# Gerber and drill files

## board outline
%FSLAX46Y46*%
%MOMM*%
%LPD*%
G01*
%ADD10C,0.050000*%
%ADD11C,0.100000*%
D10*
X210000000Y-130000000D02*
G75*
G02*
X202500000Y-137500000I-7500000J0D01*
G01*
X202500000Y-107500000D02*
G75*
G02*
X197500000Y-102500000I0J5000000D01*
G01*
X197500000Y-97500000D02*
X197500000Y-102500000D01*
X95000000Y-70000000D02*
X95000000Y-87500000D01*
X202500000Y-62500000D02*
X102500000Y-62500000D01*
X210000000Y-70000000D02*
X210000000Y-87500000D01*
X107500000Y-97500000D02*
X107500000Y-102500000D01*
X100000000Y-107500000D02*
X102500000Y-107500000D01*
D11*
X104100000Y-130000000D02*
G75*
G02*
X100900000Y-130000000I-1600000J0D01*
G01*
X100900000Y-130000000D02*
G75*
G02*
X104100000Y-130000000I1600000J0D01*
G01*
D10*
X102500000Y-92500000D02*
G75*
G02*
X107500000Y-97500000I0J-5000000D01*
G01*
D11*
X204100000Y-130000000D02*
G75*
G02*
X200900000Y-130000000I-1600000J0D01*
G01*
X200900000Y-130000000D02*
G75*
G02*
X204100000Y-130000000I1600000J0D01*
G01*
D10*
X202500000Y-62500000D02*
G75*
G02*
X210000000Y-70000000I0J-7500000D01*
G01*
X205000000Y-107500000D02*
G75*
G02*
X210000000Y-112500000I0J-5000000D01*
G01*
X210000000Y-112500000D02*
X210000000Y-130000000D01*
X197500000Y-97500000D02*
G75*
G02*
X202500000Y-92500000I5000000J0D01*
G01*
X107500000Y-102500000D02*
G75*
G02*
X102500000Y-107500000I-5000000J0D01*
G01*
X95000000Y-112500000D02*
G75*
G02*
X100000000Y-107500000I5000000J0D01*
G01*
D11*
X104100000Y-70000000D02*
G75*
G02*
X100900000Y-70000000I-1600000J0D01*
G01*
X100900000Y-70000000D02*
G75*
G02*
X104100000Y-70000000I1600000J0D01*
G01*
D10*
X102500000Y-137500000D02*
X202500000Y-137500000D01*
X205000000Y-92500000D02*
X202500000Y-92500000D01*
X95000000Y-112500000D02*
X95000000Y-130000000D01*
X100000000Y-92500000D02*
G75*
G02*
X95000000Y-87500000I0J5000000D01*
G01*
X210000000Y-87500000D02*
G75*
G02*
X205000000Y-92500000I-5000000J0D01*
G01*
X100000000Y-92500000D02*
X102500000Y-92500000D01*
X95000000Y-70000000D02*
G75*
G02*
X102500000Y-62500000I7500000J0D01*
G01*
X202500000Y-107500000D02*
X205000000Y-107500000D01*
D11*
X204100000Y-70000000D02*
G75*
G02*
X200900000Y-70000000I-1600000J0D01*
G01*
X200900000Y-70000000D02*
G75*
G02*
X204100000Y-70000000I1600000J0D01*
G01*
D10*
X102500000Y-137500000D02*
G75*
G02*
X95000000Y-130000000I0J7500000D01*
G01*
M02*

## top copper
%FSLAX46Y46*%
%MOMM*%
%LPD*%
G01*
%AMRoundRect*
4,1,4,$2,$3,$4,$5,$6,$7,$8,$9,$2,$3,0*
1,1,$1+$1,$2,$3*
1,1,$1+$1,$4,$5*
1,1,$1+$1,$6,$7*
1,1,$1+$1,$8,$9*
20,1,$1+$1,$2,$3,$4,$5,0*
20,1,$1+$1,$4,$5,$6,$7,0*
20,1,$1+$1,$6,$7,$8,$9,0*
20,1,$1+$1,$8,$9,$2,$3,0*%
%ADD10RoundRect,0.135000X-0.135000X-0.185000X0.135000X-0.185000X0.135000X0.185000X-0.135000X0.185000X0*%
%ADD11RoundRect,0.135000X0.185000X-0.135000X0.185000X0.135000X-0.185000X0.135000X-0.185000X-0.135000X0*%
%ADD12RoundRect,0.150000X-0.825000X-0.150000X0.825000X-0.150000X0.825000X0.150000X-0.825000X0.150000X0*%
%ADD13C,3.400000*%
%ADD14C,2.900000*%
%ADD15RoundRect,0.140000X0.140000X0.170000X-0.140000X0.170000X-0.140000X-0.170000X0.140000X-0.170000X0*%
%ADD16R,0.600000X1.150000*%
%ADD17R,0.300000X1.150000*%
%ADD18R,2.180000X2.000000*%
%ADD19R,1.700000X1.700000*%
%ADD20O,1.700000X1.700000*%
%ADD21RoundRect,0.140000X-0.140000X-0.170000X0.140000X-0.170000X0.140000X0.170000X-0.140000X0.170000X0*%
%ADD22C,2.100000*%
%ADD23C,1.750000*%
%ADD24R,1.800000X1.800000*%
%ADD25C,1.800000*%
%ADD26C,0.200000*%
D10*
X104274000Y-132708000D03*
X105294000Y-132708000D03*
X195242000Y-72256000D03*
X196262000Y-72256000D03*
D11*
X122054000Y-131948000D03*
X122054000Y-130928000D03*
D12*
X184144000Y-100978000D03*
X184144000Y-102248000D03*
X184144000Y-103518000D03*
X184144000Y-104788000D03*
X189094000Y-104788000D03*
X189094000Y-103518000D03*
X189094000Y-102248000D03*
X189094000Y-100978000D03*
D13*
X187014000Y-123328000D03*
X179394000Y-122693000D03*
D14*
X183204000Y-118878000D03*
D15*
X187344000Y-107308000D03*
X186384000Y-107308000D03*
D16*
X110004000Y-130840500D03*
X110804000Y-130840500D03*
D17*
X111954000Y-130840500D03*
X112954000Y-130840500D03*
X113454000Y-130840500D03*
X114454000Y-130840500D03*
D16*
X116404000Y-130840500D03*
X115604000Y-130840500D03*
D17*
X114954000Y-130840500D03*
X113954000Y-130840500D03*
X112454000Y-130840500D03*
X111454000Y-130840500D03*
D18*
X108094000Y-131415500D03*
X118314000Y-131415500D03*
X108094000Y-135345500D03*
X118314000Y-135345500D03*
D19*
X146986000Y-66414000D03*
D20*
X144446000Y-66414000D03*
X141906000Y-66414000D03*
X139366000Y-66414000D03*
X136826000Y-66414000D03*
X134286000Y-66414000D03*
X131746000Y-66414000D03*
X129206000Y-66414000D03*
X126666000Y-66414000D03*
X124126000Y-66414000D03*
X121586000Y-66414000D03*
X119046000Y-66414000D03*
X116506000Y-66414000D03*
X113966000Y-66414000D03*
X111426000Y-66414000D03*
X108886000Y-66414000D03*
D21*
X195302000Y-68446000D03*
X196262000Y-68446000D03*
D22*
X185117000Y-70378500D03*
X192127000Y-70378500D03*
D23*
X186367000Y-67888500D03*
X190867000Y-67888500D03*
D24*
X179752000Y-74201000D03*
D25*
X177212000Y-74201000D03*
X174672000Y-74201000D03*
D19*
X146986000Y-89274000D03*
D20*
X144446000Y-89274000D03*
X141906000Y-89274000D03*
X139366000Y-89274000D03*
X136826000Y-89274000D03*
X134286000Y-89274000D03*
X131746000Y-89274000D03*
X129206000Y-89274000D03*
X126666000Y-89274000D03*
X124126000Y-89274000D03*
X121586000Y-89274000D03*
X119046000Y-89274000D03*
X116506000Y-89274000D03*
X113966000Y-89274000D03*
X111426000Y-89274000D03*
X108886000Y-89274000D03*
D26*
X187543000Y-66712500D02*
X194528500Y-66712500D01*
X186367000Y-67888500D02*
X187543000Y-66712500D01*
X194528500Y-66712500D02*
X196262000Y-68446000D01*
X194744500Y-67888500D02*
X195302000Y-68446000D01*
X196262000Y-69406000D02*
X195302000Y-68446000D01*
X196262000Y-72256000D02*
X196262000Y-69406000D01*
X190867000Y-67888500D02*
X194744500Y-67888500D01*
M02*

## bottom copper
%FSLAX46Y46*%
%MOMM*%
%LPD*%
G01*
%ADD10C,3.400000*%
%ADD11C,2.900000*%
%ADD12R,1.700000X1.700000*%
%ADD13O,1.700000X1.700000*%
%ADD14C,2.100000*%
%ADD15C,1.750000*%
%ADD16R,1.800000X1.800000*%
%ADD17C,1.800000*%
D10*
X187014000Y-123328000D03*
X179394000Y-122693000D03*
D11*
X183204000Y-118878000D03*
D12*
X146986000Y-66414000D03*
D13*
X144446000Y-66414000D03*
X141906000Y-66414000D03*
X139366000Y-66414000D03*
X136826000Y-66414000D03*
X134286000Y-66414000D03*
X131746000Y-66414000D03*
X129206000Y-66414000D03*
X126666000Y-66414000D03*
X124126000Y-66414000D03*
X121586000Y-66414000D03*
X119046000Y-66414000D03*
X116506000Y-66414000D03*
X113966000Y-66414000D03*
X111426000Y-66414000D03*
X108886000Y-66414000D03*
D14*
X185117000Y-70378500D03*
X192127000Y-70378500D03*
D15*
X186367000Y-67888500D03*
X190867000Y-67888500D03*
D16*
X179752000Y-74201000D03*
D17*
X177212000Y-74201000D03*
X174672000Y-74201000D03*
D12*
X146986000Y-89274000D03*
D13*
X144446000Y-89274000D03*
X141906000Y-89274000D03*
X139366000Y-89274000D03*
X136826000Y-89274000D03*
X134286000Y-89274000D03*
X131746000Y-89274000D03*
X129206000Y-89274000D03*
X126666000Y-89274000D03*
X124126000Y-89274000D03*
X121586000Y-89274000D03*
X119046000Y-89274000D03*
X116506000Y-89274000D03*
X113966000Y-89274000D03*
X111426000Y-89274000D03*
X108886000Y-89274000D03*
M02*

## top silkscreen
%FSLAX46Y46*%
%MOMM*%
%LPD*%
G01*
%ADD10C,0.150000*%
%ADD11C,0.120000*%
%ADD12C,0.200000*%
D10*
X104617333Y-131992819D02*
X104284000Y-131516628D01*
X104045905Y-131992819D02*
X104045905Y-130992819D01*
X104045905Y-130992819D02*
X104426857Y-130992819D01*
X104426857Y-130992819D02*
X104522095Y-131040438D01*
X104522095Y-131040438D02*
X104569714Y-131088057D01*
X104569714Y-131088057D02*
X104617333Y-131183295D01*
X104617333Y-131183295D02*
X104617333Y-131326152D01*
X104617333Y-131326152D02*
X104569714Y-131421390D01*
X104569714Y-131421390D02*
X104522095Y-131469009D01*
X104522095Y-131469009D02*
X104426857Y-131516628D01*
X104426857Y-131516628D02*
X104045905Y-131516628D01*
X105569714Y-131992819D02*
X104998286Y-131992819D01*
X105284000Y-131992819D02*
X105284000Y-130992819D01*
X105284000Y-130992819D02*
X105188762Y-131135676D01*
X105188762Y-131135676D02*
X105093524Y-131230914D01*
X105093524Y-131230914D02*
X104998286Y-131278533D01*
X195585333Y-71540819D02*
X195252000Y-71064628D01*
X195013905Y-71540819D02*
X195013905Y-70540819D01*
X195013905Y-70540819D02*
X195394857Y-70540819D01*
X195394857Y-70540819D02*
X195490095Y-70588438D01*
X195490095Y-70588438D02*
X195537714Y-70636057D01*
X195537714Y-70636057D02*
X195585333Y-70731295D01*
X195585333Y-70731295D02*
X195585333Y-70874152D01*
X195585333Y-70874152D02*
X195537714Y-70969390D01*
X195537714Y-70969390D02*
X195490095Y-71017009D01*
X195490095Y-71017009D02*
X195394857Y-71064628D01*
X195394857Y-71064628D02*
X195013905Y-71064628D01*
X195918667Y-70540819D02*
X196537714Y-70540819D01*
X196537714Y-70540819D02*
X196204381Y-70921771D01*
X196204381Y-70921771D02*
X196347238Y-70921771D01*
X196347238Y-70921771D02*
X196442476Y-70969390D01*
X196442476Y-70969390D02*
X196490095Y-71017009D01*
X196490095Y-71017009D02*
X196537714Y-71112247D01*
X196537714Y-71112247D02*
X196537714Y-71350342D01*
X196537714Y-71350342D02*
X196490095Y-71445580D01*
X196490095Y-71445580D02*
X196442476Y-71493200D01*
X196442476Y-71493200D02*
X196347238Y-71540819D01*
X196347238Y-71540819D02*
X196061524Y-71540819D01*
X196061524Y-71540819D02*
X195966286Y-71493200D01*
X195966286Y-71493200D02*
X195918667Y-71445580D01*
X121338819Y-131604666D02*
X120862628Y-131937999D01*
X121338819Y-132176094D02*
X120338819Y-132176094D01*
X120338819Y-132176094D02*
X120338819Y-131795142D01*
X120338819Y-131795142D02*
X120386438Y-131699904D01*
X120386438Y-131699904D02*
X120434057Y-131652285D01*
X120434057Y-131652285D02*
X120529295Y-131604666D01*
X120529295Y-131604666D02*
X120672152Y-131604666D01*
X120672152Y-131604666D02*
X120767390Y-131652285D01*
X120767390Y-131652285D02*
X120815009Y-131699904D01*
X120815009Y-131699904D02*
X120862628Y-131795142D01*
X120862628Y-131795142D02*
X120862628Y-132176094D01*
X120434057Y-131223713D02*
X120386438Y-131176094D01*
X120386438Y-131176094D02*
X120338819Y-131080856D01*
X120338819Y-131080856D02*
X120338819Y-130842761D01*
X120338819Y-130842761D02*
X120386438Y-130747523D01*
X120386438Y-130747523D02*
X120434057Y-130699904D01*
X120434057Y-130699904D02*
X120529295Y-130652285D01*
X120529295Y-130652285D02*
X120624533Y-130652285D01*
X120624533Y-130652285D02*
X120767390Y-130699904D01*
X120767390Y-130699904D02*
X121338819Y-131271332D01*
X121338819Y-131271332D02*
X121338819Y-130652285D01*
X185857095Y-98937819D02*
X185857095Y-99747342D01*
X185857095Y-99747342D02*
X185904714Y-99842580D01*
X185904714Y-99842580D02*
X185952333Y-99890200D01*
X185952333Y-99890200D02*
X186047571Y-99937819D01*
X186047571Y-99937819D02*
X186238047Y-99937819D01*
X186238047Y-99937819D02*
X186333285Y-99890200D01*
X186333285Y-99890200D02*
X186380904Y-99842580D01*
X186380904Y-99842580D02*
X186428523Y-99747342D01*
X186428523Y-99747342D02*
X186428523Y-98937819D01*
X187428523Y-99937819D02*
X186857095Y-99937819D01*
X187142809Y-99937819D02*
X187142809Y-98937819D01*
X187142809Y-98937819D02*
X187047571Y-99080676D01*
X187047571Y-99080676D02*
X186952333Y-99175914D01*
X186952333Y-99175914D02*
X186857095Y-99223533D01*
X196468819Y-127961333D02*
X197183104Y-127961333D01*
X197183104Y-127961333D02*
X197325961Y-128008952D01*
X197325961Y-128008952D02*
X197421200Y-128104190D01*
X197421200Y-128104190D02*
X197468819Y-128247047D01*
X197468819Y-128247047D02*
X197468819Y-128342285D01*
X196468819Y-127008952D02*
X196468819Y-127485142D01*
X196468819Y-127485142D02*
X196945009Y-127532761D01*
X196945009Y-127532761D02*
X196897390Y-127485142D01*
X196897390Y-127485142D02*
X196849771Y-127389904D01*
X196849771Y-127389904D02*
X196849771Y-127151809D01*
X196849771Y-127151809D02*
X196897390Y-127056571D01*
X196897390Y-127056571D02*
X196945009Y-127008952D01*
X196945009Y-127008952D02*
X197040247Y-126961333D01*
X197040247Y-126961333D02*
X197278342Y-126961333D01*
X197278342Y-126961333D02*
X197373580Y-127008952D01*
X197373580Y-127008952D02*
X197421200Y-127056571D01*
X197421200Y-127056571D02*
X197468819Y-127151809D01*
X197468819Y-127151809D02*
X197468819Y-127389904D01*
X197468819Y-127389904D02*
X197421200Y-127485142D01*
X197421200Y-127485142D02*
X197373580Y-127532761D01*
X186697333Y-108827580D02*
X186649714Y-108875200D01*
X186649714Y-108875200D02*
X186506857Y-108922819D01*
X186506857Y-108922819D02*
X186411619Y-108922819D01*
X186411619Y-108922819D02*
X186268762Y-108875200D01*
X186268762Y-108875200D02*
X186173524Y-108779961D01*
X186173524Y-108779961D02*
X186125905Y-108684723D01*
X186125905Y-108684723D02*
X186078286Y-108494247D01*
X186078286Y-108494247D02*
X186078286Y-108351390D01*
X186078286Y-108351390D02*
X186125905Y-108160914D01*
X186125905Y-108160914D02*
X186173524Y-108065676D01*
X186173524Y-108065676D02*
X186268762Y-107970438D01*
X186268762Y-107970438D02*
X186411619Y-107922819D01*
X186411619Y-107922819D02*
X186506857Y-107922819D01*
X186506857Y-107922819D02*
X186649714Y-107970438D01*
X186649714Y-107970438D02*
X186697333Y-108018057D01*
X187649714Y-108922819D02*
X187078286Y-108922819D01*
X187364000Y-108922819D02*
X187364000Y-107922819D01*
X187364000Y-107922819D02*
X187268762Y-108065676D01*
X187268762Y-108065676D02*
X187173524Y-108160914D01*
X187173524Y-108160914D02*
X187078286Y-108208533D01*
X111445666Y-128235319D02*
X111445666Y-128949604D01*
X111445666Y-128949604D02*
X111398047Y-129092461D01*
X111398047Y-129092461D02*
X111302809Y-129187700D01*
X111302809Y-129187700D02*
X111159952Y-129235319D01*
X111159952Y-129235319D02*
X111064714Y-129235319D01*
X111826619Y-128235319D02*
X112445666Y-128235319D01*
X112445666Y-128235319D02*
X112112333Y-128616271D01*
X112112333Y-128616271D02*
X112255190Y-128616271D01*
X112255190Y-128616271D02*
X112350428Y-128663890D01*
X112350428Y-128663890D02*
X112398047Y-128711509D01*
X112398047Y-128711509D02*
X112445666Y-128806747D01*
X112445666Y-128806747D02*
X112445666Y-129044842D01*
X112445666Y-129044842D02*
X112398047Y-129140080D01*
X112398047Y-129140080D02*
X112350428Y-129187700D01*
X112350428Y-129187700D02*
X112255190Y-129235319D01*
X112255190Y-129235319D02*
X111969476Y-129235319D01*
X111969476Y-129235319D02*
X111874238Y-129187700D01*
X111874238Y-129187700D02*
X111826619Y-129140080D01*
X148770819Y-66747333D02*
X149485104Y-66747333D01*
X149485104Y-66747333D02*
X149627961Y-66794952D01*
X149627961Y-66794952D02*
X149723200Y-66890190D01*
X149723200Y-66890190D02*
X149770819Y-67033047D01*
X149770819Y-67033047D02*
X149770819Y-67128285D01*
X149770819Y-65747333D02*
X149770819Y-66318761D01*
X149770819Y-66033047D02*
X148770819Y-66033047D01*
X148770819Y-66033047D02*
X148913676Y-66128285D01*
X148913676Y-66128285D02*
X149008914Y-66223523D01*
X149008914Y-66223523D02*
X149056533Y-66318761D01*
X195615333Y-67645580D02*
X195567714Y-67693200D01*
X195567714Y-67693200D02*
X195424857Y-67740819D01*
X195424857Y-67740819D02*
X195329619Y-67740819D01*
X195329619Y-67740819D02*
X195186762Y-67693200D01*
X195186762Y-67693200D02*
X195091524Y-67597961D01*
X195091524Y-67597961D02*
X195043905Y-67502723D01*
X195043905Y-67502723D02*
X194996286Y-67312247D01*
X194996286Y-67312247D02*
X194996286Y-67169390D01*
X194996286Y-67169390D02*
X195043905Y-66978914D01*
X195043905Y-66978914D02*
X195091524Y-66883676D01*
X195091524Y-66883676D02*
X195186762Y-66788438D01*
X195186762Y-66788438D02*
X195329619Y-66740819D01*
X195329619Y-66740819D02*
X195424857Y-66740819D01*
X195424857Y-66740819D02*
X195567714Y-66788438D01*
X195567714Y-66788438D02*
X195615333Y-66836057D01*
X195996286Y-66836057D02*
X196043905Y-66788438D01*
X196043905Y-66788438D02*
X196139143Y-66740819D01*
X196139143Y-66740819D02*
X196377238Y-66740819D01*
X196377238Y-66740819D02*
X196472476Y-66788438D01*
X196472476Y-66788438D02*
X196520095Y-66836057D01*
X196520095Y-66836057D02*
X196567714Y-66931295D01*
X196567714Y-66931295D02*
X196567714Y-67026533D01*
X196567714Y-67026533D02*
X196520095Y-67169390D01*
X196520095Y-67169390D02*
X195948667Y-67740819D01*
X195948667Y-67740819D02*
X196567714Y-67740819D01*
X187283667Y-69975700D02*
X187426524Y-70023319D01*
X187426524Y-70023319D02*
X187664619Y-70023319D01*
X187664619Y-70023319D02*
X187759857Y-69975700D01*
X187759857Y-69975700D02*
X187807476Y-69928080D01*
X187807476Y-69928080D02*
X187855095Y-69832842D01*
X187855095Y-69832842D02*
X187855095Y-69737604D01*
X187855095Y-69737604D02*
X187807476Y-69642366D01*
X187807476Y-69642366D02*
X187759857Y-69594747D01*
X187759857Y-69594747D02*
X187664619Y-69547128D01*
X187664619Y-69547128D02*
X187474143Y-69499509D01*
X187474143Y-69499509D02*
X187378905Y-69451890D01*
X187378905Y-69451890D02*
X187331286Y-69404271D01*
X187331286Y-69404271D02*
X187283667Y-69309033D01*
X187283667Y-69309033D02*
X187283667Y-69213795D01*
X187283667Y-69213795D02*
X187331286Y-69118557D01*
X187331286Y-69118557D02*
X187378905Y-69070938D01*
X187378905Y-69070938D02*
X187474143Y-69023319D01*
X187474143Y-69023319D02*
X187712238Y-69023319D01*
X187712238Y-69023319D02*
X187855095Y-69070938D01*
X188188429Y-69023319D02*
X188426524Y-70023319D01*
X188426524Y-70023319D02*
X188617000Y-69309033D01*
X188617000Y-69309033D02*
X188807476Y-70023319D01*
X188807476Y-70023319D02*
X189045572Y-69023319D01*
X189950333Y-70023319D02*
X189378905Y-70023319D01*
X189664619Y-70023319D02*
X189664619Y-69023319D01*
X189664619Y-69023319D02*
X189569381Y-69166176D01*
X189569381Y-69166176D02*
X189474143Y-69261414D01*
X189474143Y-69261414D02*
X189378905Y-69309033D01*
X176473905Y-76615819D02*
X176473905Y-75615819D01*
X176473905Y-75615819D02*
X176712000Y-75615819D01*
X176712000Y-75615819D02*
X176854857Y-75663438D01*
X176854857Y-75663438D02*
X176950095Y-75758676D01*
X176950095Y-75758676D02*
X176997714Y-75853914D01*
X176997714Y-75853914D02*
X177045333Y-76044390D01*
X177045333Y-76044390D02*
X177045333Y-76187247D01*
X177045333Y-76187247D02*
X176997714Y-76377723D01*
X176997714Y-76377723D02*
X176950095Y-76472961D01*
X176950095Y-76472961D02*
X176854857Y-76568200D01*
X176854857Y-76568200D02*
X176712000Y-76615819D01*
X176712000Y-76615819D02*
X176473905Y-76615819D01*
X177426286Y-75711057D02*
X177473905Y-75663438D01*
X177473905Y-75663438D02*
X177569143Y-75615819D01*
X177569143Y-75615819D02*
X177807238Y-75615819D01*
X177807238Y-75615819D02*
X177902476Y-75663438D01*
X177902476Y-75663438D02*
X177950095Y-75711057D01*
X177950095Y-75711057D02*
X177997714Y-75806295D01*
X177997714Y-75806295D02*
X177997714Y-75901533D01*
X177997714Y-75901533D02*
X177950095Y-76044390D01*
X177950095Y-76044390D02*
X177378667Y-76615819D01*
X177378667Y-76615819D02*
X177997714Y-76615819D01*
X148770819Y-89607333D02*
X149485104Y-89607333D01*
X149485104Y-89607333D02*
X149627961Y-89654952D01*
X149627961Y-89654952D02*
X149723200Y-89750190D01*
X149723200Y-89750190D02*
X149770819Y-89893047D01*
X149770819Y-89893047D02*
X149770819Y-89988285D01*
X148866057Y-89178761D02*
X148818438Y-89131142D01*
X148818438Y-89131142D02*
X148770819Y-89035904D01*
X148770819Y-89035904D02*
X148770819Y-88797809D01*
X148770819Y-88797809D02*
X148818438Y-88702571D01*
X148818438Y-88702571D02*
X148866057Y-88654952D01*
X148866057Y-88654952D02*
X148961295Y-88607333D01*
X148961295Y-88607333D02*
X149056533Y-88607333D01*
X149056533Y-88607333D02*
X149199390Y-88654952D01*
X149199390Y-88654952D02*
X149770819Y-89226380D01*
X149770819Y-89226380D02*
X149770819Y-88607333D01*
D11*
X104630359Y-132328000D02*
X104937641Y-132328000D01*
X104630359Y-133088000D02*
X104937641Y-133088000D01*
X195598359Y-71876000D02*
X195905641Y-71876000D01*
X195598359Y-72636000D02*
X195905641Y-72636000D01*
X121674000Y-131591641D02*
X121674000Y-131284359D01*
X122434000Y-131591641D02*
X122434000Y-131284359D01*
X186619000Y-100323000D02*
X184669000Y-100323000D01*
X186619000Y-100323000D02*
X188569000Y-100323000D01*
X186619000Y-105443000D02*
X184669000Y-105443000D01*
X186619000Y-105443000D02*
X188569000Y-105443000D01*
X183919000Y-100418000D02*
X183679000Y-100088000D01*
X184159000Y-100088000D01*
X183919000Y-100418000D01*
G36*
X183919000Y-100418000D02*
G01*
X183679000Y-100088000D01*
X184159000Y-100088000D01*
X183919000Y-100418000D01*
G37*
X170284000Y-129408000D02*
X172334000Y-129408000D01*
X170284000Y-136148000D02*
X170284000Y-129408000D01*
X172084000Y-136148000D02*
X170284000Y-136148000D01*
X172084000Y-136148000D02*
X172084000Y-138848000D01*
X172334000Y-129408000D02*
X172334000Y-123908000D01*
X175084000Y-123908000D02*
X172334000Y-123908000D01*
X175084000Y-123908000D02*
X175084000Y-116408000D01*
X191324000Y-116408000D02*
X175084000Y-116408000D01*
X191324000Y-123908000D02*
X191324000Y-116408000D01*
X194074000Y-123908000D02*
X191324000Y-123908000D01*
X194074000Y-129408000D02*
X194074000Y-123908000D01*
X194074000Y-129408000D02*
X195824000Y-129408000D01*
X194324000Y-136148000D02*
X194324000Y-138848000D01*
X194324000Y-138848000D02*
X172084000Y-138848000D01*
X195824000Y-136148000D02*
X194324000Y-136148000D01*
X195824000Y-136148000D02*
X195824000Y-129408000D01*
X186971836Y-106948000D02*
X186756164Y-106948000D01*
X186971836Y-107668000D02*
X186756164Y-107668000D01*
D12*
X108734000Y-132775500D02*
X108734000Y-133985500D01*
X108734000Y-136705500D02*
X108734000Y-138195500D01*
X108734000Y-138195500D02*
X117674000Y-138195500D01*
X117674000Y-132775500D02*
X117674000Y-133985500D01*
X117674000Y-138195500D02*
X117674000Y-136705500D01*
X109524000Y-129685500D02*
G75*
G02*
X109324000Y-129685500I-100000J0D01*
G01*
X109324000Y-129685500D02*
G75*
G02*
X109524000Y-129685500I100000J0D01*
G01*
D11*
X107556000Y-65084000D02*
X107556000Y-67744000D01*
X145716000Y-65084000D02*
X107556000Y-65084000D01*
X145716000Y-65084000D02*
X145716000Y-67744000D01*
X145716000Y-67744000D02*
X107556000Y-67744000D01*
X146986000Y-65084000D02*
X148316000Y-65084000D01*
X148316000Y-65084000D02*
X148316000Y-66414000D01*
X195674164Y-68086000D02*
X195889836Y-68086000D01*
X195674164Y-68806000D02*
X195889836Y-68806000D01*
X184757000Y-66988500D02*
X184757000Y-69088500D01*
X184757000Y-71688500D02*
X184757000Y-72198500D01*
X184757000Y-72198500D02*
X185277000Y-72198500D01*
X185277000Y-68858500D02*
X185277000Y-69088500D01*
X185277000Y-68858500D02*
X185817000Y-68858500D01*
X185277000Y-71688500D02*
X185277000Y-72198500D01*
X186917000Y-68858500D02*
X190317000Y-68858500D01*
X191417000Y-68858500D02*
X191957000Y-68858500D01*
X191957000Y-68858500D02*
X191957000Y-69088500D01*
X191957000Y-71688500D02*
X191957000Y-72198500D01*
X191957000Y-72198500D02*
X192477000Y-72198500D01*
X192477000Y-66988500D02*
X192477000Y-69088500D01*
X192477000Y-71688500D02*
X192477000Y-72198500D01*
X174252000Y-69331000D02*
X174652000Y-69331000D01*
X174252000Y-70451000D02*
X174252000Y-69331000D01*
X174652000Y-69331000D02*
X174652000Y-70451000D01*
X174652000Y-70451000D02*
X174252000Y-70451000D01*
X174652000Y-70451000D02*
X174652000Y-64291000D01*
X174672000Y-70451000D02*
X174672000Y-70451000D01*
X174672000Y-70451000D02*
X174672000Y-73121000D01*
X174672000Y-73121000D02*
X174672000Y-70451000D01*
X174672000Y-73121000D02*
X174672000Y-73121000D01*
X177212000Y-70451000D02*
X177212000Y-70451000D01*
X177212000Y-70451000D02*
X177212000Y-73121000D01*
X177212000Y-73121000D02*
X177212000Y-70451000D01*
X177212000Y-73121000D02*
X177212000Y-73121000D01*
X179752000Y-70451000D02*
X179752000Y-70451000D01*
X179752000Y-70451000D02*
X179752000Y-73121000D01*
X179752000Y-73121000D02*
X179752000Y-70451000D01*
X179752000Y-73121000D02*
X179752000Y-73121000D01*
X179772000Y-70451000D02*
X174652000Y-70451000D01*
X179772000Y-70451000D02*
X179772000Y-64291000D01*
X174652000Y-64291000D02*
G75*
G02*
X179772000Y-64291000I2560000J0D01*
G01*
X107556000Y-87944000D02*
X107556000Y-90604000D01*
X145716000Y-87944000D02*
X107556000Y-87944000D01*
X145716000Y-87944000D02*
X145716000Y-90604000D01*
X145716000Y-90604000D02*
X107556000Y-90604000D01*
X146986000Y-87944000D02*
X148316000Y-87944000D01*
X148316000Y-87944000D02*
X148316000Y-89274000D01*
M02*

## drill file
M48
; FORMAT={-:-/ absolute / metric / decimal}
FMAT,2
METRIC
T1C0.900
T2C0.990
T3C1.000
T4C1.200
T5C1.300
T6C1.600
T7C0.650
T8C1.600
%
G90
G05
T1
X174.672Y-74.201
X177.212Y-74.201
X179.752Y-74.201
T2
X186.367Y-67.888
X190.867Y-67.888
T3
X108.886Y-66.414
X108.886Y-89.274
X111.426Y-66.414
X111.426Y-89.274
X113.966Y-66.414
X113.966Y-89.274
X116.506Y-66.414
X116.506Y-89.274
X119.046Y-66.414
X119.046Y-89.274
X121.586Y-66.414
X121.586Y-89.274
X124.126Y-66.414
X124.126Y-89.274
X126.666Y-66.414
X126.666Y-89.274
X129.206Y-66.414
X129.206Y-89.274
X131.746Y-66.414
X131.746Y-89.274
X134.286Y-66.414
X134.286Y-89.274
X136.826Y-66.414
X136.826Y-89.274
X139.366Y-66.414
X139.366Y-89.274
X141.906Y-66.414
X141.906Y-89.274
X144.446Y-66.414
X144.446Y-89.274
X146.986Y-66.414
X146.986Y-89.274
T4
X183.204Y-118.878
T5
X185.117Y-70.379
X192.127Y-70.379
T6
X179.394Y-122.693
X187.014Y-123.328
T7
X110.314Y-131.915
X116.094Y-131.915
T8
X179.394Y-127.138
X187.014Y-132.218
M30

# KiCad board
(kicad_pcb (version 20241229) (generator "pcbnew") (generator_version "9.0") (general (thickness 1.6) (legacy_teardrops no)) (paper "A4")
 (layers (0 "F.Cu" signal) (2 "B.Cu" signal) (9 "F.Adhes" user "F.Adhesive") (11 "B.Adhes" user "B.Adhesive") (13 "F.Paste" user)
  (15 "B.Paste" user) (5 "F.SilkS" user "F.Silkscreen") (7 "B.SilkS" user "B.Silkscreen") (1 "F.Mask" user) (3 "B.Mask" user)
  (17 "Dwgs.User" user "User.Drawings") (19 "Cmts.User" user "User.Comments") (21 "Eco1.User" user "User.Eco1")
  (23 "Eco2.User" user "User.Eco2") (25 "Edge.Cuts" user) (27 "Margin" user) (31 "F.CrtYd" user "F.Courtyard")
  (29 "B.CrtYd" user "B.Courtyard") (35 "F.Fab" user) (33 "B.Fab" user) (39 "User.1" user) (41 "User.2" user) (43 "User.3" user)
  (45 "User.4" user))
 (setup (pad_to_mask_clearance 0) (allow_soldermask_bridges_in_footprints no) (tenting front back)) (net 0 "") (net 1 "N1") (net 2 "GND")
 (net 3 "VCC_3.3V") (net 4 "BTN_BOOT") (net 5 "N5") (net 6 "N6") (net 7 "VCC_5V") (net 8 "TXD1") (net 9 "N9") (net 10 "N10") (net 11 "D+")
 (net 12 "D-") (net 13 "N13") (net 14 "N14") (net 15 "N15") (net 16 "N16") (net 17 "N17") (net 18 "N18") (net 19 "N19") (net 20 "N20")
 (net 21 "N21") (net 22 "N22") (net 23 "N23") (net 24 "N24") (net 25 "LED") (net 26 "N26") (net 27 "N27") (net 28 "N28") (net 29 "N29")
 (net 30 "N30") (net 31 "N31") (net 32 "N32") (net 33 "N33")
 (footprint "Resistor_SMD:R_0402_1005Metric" (layer "F.Cu") (at 104.784 132.708)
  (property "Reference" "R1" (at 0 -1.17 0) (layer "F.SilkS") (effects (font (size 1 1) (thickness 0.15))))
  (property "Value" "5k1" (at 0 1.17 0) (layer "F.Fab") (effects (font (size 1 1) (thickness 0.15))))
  (fp_line (start -0.153641 -0.38) (end 0.153641 -0.38) (stroke (width 0.12) (type solid)) (layer "F.SilkS"))
  (fp_line (start -0.153641 0.38) (end 0.153641 0.38) (stroke (width 0.12) (type solid)) (layer "F.SilkS"))
  (pad "1" smd roundrect (at -0.51 0) (size 0.54 0.64) (layers "F.Cu" "F.Mask" "F.Paste") (roundrect_rratio 0.25) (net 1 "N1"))
  (pad "2" smd roundrect (at 0.51 0) (size 0.54 0.64) (layers "F.Cu" "F.Mask" "F.Paste") (roundrect_rratio 0.25) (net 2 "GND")))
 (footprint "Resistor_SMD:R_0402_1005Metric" (layer "F.Cu") (at 195.752 72.256)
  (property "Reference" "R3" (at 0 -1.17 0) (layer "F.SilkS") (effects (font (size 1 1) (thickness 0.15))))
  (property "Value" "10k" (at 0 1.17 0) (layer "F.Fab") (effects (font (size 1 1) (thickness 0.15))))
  (fp_line (start -0.153641 -0.38) (end 0.153641 -0.38) (stroke (width 0.12) (type solid)) (layer "F.SilkS"))
  (fp_line (start -0.153641 0.38) (end 0.153641 0.38) (stroke (width 0.12) (type solid)) (layer "F.SilkS"))
  (pad "1" smd roundrect (at -0.51 0) (size 0.54 0.64) (layers "F.Cu" "F.Mask" "F.Paste") (roundrect_rratio 0.25) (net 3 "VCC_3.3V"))
  (pad "2" smd roundrect (at 0.51 0) (size 0.54 0.64) (layers "F.Cu" "F.Mask" "F.Paste") (roundrect_rratio 0.25) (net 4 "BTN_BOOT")))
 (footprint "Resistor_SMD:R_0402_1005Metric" (layer "F.Cu") (at 122.054 131.438 90)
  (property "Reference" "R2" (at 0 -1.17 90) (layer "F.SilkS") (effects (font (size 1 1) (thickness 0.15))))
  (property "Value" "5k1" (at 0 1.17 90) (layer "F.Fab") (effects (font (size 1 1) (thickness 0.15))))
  (fp_line (start -0.153641 -0.38) (end 0.153641 -0.38) (stroke (width 0.12) (type solid)) (layer "F.SilkS"))
  (fp_line (start -0.153641 0.38) (end 0.153641 0.38) (stroke (width 0.12) (type solid)) (layer "F.SilkS"))
  (pad "1" smd roundrect (at -0.51 0 90) (size 0.54 0.64) (layers "F.Cu" "F.Mask" "F.Paste") (roundrect_rratio 0.25) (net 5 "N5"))
  (pad "2" smd roundrect (at 0.51 0 90) (size 0.54 0.64) (layers "F.Cu" "F.Mask" "F.Paste") (roundrect_rratio 0.25) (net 2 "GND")))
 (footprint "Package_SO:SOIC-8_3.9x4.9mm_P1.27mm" (layer "F.Cu") (at 186.619 102.883)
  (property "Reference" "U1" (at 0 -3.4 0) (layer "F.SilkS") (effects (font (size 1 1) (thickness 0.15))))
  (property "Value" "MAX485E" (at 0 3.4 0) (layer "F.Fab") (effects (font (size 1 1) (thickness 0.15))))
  (fp_line (start 0 -2.56) (end -1.95 -2.56) (stroke (width 0.12) (type solid)) (layer "F.SilkS"))
  (fp_line (start 0 -2.56) (end 1.95 -2.56) (stroke (width 0.12) (type solid)) (layer "F.SilkS"))
  (fp_line (start 0 2.56) (end -1.95 2.56) (stroke (width 0.12) (type solid)) (layer "F.SilkS"))
  (fp_line (start 0 2.56) (end 1.95 2.56) (stroke (width 0.12) (type solid)) (layer "F.SilkS"))
  (fp_poly
   (pts (xy -2.7 -2.465) (xy -2.94 -2.795) (xy -2.46 -2.795) (xy -2.7 -2.465)) (stroke (width 0.12) (type solid)) (fill yes)
   (layer "F.SilkS"))
  (pad "1" smd roundrect (at -2.475 -1.905) (size 1.95 0.6) (layers "F.Cu" "F.Mask" "F.Paste") (roundrect_rratio 0.25) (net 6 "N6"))
  (pad "2" smd roundrect (at -2.475 -0.635) (size 1.95 0.6) (layers "F.Cu" "F.Mask" "F.Paste") (roundrect_rratio 0.25) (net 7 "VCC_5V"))
  (pad "3" smd roundrect (at -2.475 0.635) (size 1.95 0.6) (layers "F.Cu" "F.Mask" "F.Paste") (roundrect_rratio 0.25) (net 7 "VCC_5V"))
  (pad "4" smd roundrect (at -2.475 1.905) (size 1.95 0.6) (layers "F.Cu" "F.Mask" "F.Paste") (roundrect_rratio 0.25) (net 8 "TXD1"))
  (pad "5" smd roundrect (at 2.475 1.905) (size 1.95 0.6) (layers "F.Cu" "F.Mask" "F.Paste") (roundrect_rratio 0.25) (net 2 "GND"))
  (pad "6" smd roundrect (at 2.475 0.635) (size 1.95 0.6) (layers "F.Cu" "F.Mask" "F.Paste") (roundrect_rratio 0.25) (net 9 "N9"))
  (pad "7" smd roundrect (at 2.475 -0.635) (size 1.95 0.6) (layers "F.Cu" "F.Mask" "F.Paste") (roundrect_rratio 0.25) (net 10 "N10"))
  (pad "8" smd roundrect (at 2.475 -1.905) (size 1.95 0.6) (layers "F.Cu" "F.Mask" "F.Paste") (roundrect_rratio 0.25) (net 7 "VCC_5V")))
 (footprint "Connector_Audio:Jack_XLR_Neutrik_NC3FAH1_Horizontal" (layer "F.Cu") (at 187.014 123.328 -90)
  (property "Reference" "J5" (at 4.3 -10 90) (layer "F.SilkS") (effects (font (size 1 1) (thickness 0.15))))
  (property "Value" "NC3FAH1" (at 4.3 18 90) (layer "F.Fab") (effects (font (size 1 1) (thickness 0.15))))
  (fp_line (start 6.08 16.73) (end 6.08 14.68) (stroke (width 0.12) (type solid)) (layer "F.SilkS"))
  (fp_line (start 12.82 16.73) (end 6.08 16.73) (stroke (width 0.12) (type solid)) (layer "F.SilkS"))
  (fp_line (start 12.82 14.93) (end 12.82 16.73) (stroke (width 0.12) (type solid)) (layer "F.SilkS"))
  (fp_line (start 12.82 14.93) (end 15.52 14.93) (stroke (width 0.12) (type solid)) (layer "F.SilkS"))
  (fp_line (start 6.08 14.68) (end 0.58 14.68) (stroke (width 0.12) (type solid)) (layer "F.SilkS"))
  (fp_line (start 0.58 11.93) (end 0.58 14.68) (stroke (width 0.12) (type solid)) (layer "F.SilkS"))
  (fp_line (start 0.58 11.93) (end -6.92 11.93) (stroke (width 0.12) (type solid)) (layer "F.SilkS"))
  (fp_line (start -6.92 -4.31) (end -6.92 11.93) (stroke (width 0.12) (type solid)) (layer "F.SilkS"))
  (fp_line (start 0.58 -4.31) (end -6.92 -4.31) (stroke (width 0.12) (type solid)) (layer "F.SilkS"))
  (fp_line (start 0.58 -7.06) (end 0.58 -4.31) (stroke (width 0.12) (type solid)) (layer "F.SilkS"))
  (fp_line (start 6.08 -7.06) (end 0.58 -7.06) (stroke (width 0.12) (type solid)) (layer "F.SilkS"))
  (fp_line (start 6.08 -7.06) (end 6.08 -8.81) (stroke (width 0.12) (type solid)) (layer "F.SilkS"))
  (fp_line (start 12.82 -7.31) (end 15.52 -7.31) (stroke (width 0.12) (type solid)) (layer "F.SilkS"))
  (fp_line (start 15.52 -7.31) (end 15.52 14.93) (stroke (width 0.12) (type solid)) (layer "F.SilkS"))
  (fp_line (start 12.82 -8.81) (end 12.82 -7.31) (stroke (width 0.12) (type solid)) (layer "F.SilkS"))
  (fp_line (start 12.82 -8.81) (end 6.08 -8.81) (stroke (width 0.12) (type solid)) (layer "F.SilkS"))
  (pad "" np_thru_hole circle (at 3.81 7.62 270) (size 1.6 1.6) (drill 1.6) (layers "*.Cu" "*.Mask"))
  (pad "" np_thru_hole circle (at 8.89 0 270) (size 1.6 1.6) (drill 1.6) (layers "*.Cu" "*.Mask"))
  (pad "1" thru_hole circle (at 0 0 270) (size 3.4 3.4) (drill 1.6) (layers "*.Cu" "*.Mask") (remove_unused_layers no) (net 2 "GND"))
  (pad "2" thru_hole circle (at -0.635 7.62 270) (size 3.4 3.4) (drill 1.6) (layers "*.Cu" "*.Mask") (remove_unused_layers no)
   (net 10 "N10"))
  (pad "3" thru_hole circle (at -4.45 3.81 270) (size 2.9 2.9) (drill 1.2) (layers "*.Cu" "*.Mask") (remove_unused_layers no) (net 9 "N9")))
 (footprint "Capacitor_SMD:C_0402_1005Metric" (layer "F.Cu") (at 186.864 107.308 180)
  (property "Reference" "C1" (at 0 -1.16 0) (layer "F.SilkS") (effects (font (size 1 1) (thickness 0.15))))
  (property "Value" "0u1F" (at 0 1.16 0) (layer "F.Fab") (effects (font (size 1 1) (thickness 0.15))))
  (fp_line (start -0.107836 0.36) (end 0.107836 0.36) (stroke (width 0.12) (type solid)) (layer "F.SilkS"))
  (fp_line (start -0.107836 -0.36) (end 0.107836 -0.36) (stroke (width 0.12) (type solid)) (layer "F.SilkS"))
  (pad "1" smd roundrect (at -0.48 0 180) (size 0.56 0.62) (layers "F.Cu" "F.Mask" "F.Paste") (roundrect_rratio 0.25) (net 7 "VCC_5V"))
  (pad "2" smd roundrect (at 0.48 0 180) (size 0.56 0.62) (layers "F.Cu" "F.Mask" "F.Paste") (roundrect_rratio 0.25) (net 2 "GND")))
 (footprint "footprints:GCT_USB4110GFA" (layer "F.Cu") (at 113.204 131.9155)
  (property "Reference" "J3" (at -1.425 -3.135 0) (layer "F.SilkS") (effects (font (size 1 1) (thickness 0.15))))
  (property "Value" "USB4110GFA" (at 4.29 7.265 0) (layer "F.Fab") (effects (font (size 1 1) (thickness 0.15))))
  (fp_line (start -4.47 0.86) (end -4.47 2.07) (stroke (width 0.2) (type solid)) (layer "F.SilkS"))
  (fp_line (start -4.47 4.79) (end -4.47 6.28) (stroke (width 0.2) (type solid)) (layer "F.SilkS"))
  (fp_line (start -4.47 6.28) (end 4.47 6.28) (stroke (width 0.2) (type solid)) (layer "F.SilkS"))
  (fp_line (start 4.47 0.86) (end 4.47 2.07) (stroke (width 0.2) (type solid)) (layer "F.SilkS"))
  (fp_line (start 4.47 6.28) (end 4.47 4.79) (stroke (width 0.2) (type solid)) (layer "F.SilkS"))
  (fp_circle (center -3.78 -2.23) (end -3.68 -2.23) (stroke (width 0.2) (type solid)) (fill no) (layer "F.SilkS"))
  (pad "" np_thru_hole circle (at -2.89 0) (size 0.65 0.65) (drill 0.65) (layers "*.Cu" "*.Mask"))
  (pad "" np_thru_hole circle (at 2.89 0) (size 0.65 0.65) (drill 0.65) (layers "*.Cu" "*.Mask"))
  (pad "A1/B12" smd rect (at -3.2 -1.075) (size 0.6 1.15) (layers "F.Cu" "F.Mask" "F.Paste") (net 2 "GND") (solder_mask_margin 0.102))
  (pad "A4/B9" smd rect (at -2.4 -1.075) (size 0.6 1.15) (layers "F.Cu" "F.Mask" "F.Paste") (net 7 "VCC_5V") (solder_mask_margin 0.102))
  (pad "A5" smd rect (at -1.25 -1.075) (size 0.3 1.15) (layers "F.Cu" "F.Mask" "F.Paste") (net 1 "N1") (solder_mask_margin 0.102))
  (pad "A6" smd rect (at -0.25 -1.075) (size 0.3 1.15) (layers "F.Cu" "F.Mask" "F.Paste") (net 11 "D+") (solder_mask_margin 0.102))
  (pad "A7" smd rect (at 0.25 -1.075) (size 0.3 1.15) (layers "F.Cu" "F.Mask" "F.Paste") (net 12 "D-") (solder_mask_margin 0.102))
  (pad "A8" smd rect (at 1.25 -1.075) (size 0.3 1.15) (layers "F.Cu" "F.Mask" "F.Paste") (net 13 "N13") (solder_mask_margin 0.102))
  (pad "B1/A12" smd rect (at 3.2 -1.075) (size 0.6 1.15) (layers "F.Cu" "F.Mask" "F.Paste") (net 2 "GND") (solder_mask_margin 0.102))
  (pad "B4/A9" smd rect (at 2.4 -1.075) (size 0.6 1.15) (layers "F.Cu" "F.Mask" "F.Paste") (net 7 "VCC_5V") (solder_mask_margin 0.102))
  (pad "B5" smd rect (at 1.75 -1.075) (size 0.3 1.15) (layers "F.Cu" "F.Mask" "F.Paste") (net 5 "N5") (solder_mask_margin 0.102))
  (pad "B6" smd rect (at 0.75 -1.075) (size 0.3 1.15) (layers "F.Cu" "F.Mask" "F.Paste") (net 11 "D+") (solder_mask_margin 0.102))
  (pad "B7" smd rect (at -0.75 -1.075) (size 0.3 1.15) (layers "F.Cu" "F.Mask" "F.Paste") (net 12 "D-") (solder_mask_margin 0.102))
  (pad "B8" smd rect (at -1.75 -1.075) (size 0.3 1.15) (layers "F.Cu" "F.Mask" "F.Paste") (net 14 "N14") (solder_mask_margin 0.102))
  (pad "S1" smd rect (at -5.11 -0.5) (size 2.18 2) (layers "F.Cu" "F.Mask" "F.Paste") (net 2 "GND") (solder_mask_margin 0.102))
  (pad "S2" smd rect (at 5.11 -0.5) (size 2.18 2) (layers "F.Cu" "F.Mask" "F.Paste") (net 2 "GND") (solder_mask_margin 0.102))
  (pad "S3" smd rect (at -5.11 3.43) (size 2.18 2) (layers "F.Cu" "F.Mask" "F.Paste") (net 2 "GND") (solder_mask_margin 0.102))
  (pad "S4" smd rect (at 5.11 3.43) (size 2.18 2) (layers "F.Cu" "F.Mask" "F.Paste") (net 2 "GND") (solder_mask_margin 0.102)))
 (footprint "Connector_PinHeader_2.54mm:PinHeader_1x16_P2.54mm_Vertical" (layer "F.Cu") (at 146.986 66.414 -90)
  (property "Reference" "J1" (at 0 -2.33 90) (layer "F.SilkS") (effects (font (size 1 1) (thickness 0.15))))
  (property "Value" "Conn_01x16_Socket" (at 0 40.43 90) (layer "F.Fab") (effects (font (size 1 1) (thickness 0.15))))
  (fp_line (start -1.33 39.43) (end 1.33 39.43) (stroke (width 0.12) (type solid)) (layer "F.SilkS"))
  (fp_line (start -1.33 1.27) (end -1.33 39.43) (stroke (width 0.12) (type solid)) (layer "F.SilkS"))
  (fp_line (start -1.33 1.27) (end 1.33 1.27) (stroke (width 0.12) (type solid)) (layer "F.SilkS"))
  (fp_line (start 1.33 1.27) (end 1.33 39.43) (stroke (width 0.12) (type solid)) (layer "F.SilkS"))
  (fp_line (start -1.33 0) (end -1.33 -1.33) (stroke (width 0.12) (type solid)) (layer "F.SilkS"))
  (fp_line (start -1.33 -1.33) (end 0 -1.33) (stroke (width 0.12) (type solid)) (layer "F.SilkS"))
  (pad "1" thru_hole rect (at 0 0 270) (size 1.7 1.7) (drill 1) (layers "*.Cu" "*.Mask") (remove_unused_layers no) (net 2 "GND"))
  (pad "2" thru_hole oval (at 0 2.54 270) (size 1.7 1.7) (drill 1) (layers "*.Cu" "*.Mask") (remove_unused_layers no) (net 3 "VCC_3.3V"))
  (pad "3" thru_hole oval (at 0 5.08 270) (size 1.7 1.7) (drill 1) (layers "*.Cu" "*.Mask") (remove_unused_layers no) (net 4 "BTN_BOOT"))
  (pad "4" thru_hole oval (at 0 7.62 270) (size 1.7 1.7) (drill 1) (layers "*.Cu" "*.Mask") (remove_unused_layers no) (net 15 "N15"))
  (pad "5" thru_hole oval (at 0 10.16 270) (size 1.7 1.7) (drill 1) (layers "*.Cu" "*.Mask") (remove_unused_layers no) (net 2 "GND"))
  (pad "6" thru_hole oval (at 0 12.7 270) (size 1.7 1.7) (drill 1) (layers "*.Cu" "*.Mask") (remove_unused_layers no) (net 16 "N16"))
  (pad "7" thru_hole oval (at 0 15.24 270) (size 1.7 1.7) (drill 1) (layers "*.Cu" "*.Mask") (remove_unused_layers no) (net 2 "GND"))
  (pad "8" thru_hole oval (at 0 17.78 270) (size 1.7 1.7) (drill 1) (layers "*.Cu" "*.Mask") (remove_unused_layers no) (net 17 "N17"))
  (pad "9" thru_hole oval (at 0 20.32 270) (size 1.7 1.7) (drill 1) (layers "*.Cu" "*.Mask") (remove_unused_layers no) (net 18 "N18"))
  (pad "10" thru_hole oval (at 0 22.86 270) (size 1.7 1.7) (drill 1) (layers "*.Cu" "*.Mask") (remove_unused_layers no) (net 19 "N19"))
  (pad "11" thru_hole oval (at 0 25.4 270) (size 1.7 1.7) (drill 1) (layers "*.Cu" "*.Mask") (remove_unused_layers no) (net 2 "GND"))
  (pad "12" thru_hole oval (at 0 27.94 270) (size 1.7 1.7) (drill 1) (layers "*.Cu" "*.Mask") (remove_unused_layers no) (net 8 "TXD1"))
  (pad "13" thru_hole oval (at 0 30.48 270) (size 1.7 1.7) (drill 1) (layers "*.Cu" "*.Mask") (remove_unused_layers no) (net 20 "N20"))
  (pad "14" thru_hole oval (at 0 33.02 270) (size 1.7 1.7) (drill 1) (layers "*.Cu" "*.Mask") (remove_unused_layers no) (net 2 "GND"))
  (pad "15" thru_hole oval (at 0 35.56 270) (size 1.7 1.7) (drill 1) (layers "*.Cu" "*.Mask") (remove_unused_layers no) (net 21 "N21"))
  (pad "16" thru_hole oval (at 0 38.1 270) (size 1.7 1.7) (drill 1) (layers "*.Cu" "*.Mask") (remove_unused_layers no) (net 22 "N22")))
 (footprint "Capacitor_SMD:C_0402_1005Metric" (layer "F.Cu") (at 195.782 68.446)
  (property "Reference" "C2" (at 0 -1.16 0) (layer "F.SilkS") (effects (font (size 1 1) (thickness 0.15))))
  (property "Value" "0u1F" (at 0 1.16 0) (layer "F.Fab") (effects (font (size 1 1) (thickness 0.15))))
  (fp_line (start -0.107836 -0.36) (end 0.107836 -0.36) (stroke (width 0.12) (type solid)) (layer "F.SilkS"))
  (fp_line (start -0.107836 0.36) (end 0.107836 0.36) (stroke (width 0.12) (type solid)) (layer "F.SilkS"))
  (pad "1" smd roundrect (at -0.48 0) (size 0.56 0.62) (layers "F.Cu" "F.Mask" "F.Paste") (roundrect_rratio 0.25) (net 4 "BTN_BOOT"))
  (pad "2" smd roundrect (at 0.48 0) (size 0.56 0.62) (layers "F.Cu" "F.Mask" "F.Paste") (roundrect_rratio 0.25) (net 2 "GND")))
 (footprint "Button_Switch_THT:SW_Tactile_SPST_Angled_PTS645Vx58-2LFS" (layer "F.Cu") (at 186.367 67.8885)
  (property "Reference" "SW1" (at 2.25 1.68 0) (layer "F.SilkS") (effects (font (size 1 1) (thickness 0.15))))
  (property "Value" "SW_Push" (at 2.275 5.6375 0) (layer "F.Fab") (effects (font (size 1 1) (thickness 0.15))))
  (fp_line (start -1.61 -0.9) (end -1.61 1.2) (stroke (width 0.12) (type solid)) (layer "F.SilkS"))
  (fp_line (start -1.61 3.8) (end -1.61 4.31) (stroke (width 0.12) (type solid)) (layer "F.SilkS"))
  (fp_line (start -1.61 4.31) (end -1.09 4.31) (stroke (width 0.12) (type solid)) (layer "F.SilkS"))
  (fp_line (start -1.09 0.97) (end -1.09 1.2) (stroke (width 0.12) (type solid)) (layer "F.SilkS"))
  (fp_line (start -1.09 0.97) (end -0.55 0.97) (stroke (width 0.12) (type solid)) (layer "F.SilkS"))
  (fp_line (start -1.09 3.8) (end -1.09 4.31) (stroke (width 0.12) (type solid)) (layer "F.SilkS"))
  (fp_line (start 0.55 0.97) (end 3.95 0.97) (stroke (width 0.12) (type solid)) (layer "F.SilkS"))
  (fp_line (start 5.05 0.97) (end 5.59 0.97) (stroke (width 0.12) (type solid)) (layer "F.SilkS"))
  (fp_line (start 5.59 0.97) (end 5.59 1.2) (stroke (width 0.12) (type solid)) (layer "F.SilkS"))
  (fp_line (start 5.59 3.8) (end 5.59 4.31) (stroke (width 0.12) (type solid)) (layer "F.SilkS"))
  (fp_line (start 5.59 4.31) (end 6.11 4.31) (stroke (width 0.12) (type solid)) (layer "F.SilkS"))
  (fp_line (start 6.11 -0.9) (end 6.11 1.2) (stroke (width 0.12) (type solid)) (layer "F.SilkS"))
  (fp_line (start 6.11 3.8) (end 6.11 4.31) (stroke (width 0.12) (type solid)) (layer "F.SilkS"))
  (pad "" thru_hole circle (at -1.25 2.49) (size 2.1 2.1) (drill 1.3) (layers "*.Cu" "*.Mask") (remove_unused_layers no))
  (pad "" thru_hole circle (at 5.76 2.49) (size 2.1 2.1) (drill 1.3) (layers "*.Cu" "*.Mask") (remove_unused_layers no))
  (pad "1" thru_hole circle (at 0 0) (size 1.75 1.75) (drill 0.99) (layers "*.Cu" "*.Mask") (remove_unused_layers no) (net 2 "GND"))
  (pad "2" thru_hole circle (at 4.5 0) (size 1.75 1.75) (drill 0.99) (layers "*.Cu" "*.Mask") (remove_unused_layers no) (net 4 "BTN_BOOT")))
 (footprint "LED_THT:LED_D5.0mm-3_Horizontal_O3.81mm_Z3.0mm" (layer "F.Cu") (at 179.752 74.201 180)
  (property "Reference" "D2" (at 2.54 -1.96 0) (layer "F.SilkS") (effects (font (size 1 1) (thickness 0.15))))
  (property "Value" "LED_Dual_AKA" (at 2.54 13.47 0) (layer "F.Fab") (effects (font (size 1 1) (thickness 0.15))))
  (fp_line (start 5.5 4.87) (end 5.1 4.87) (stroke (width 0.12) (type solid)) (layer "F.SilkS"))
  (fp_line (start 5.5 3.75) (end 5.5 4.87) (stroke (width 0.12) (type solid)) (layer "F.SilkS"))
  (fp_line (start 5.1 4.87) (end 5.1 3.75) (stroke (width 0.12) (type solid)) (layer "F.SilkS"))
  (fp_line (start 5.1 3.75) (end 5.5 3.75) (stroke (width 0.12) (type solid)) (layer "F.SilkS"))
  (fp_line (start 5.1 3.75) (end 5.1 9.91) (stroke (width 0.12) (type solid)) (layer "F.SilkS"))
  (fp_line (start 5.08 3.75) (end 5.08 3.75) (stroke (width 0.12) (type solid)) (layer "F.SilkS"))
  (fp_line (start 5.08 3.75) (end 5.08 1.08) (stroke (width 0.12) (type solid)) (layer "F.SilkS"))
  (fp_line (start 5.08 1.08) (end 5.08 3.75) (stroke (width 0.12) (type solid)) (layer "F.SilkS"))
  (fp_line (start 5.08 1.08) (end 5.08 1.08) (stroke (width 0.12) (type solid)) (layer "F.SilkS"))
  (fp_line (start 2.54 3.75) (end 2.54 3.75) (stroke (width 0.12) (type solid)) (layer "F.SilkS"))
  (fp_line (start 2.54 3.75) (end 2.54 1.08) (stroke (width 0.12) (type solid)) (layer "F.SilkS"))
  (fp_line (start 2.54 1.08) (end 2.54 3.75) (stroke (width 0.12) (type solid)) (layer "F.SilkS"))
  (fp_line (start 2.54 1.08) (end 2.54 1.08) (stroke (width 0.12) (type solid)) (layer "F.SilkS"))
  (fp_line (start 0 3.75) (end 0 3.75) (stroke (width 0.12) (type solid)) (layer "F.SilkS"))
  (fp_line (start 0 3.75) (end 0 1.08) (stroke (width 0.12) (type solid)) (layer "F.SilkS"))
  (fp_line (start 0 1.08) (end 0 3.75) (stroke (width 0.12) (type solid)) (layer "F.SilkS"))
  (fp_line (start 0 1.08) (end 0 1.08) (stroke (width 0.12) (type solid)) (layer "F.SilkS"))
  (fp_line (start -0.02 3.75) (end 5.1 3.75) (stroke (width 0.12) (type solid)) (layer "F.SilkS"))
  (fp_line (start -0.02 3.75) (end -0.02 9.91) (stroke (width 0.12) (type solid)) (layer "F.SilkS"))
  (fp_arc (start 5.1 9.91) (mid 2.54 12.47) (end -0.02 9.91) (stroke (width 0.12) (type solid)) (layer "F.SilkS"))
  (pad "1" thru_hole rect (at 0 0 180) (size 1.8 1.8) (drill 0.9) (layers "*.Cu" "*.Mask") (remove_unused_layers no) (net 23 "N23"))
  (pad "2" thru_hole circle (at 2.54 0 180) (size 1.8 1.8) (drill 0.9) (layers "*.Cu" "*.Mask") (remove_unused_layers no) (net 2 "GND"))
  (pad "3" thru_hole circle (at 5.08 0 180) (size 1.8 1.8) (drill 0.9) (layers "*.Cu" "*.Mask") (remove_unused_layers no) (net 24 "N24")))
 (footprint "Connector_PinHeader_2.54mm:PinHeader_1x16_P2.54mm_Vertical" (layer "F.Cu") (at 146.986 89.274 -90)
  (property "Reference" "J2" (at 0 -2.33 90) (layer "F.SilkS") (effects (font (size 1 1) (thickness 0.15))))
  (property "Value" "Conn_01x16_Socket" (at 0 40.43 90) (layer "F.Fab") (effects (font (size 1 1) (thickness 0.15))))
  (fp_line (start -1.33 39.43) (end 1.33 39.43) (stroke (width 0.12) (type solid)) (layer "F.SilkS"))
  (fp_line (start -1.33 1.27) (end -1.33 39.43) (stroke (width 0.12) (type solid)) (layer "F.SilkS"))
  (fp_line (start -1.33 1.27) (end 1.33 1.27) (stroke (width 0.12) (type solid)) (layer "F.SilkS"))
  (fp_line (start 1.33 1.27) (end 1.33 39.43) (stroke (width 0.12) (type solid)) (layer "F.SilkS"))
  (fp_line (start -1.33 0) (end -1.33 -1.33) (stroke (width 0.12) (type solid)) (layer "F.SilkS"))
  (fp_line (start -1.33 -1.33) (end 0 -1.33) (stroke (width 0.12) (type solid)) (layer "F.SilkS"))
  (pad "1" thru_hole rect (at 0 0 270) (size 1.7 1.7) (drill 1) (layers "*.Cu" "*.Mask") (remove_unused_layers no) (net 2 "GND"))
  (pad "2" thru_hole oval (at 0 2.54 270) (size 1.7 1.7) (drill 1) (layers "*.Cu" "*.Mask") (remove_unused_layers no) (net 2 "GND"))
  (pad "3" thru_hole oval (at 0 5.08 270) (size 1.7 1.7) (drill 1) (layers "*.Cu" "*.Mask") (remove_unused_layers no) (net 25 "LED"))
  (pad "4" thru_hole oval (at 0 7.62 270) (size 1.7 1.7) (drill 1) (layers "*.Cu" "*.Mask") (remove_unused_layers no) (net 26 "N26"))
  (pad "5" thru_hole oval (at 0 10.16 270) (size 1.7 1.7) (drill 1) (layers "*.Cu" "*.Mask") (remove_unused_layers no) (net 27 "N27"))
  (pad "6" thru_hole oval (at 0 12.7 270) (size 1.7 1.7) (drill 1) (layers "*.Cu" "*.Mask") (remove_unused_layers no) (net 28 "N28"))
  (pad "7" thru_hole oval (at 0 15.24 270) (size 1.7 1.7) (drill 1) (layers "*.Cu" "*.Mask") (remove_unused_layers no) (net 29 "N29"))
  (pad "8" thru_hole oval (at 0 17.78 270) (size 1.7 1.7) (drill 1) (layers "*.Cu" "*.Mask") (remove_unused_layers no) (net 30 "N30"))
  (pad "9" thru_hole oval (at 0 20.32 270) (size 1.7 1.7) (drill 1) (layers "*.Cu" "*.Mask") (remove_unused_layers no) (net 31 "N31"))
  (pad "10" thru_hole oval (at 0 22.86 270) (size 1.7 1.7) (drill 1) (layers "*.Cu" "*.Mask") (remove_unused_layers no) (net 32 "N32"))
  (pad "11" thru_hole oval (at 0 25.4 270) (size 1.7 1.7) (drill 1) (layers "*.Cu" "*.Mask") (remove_unused_layers no) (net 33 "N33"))
  (pad "12" thru_hole oval (at 0 27.94 270) (size 1.7 1.7) (drill 1) (layers "*.Cu" "*.Mask") (remove_unused_layers no) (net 2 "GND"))
  (pad "13" thru_hole oval (at 0 30.48 270) (size 1.7 1.7) (drill 1) (layers "*.Cu" "*.Mask") (remove_unused_layers no) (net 7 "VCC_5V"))
  (pad "14" thru_hole oval (at 0 33.02 270) (size 1.7 1.7) (drill 1) (layers "*.Cu" "*.Mask") (remove_unused_layers no) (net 11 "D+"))
  (pad "15" thru_hole oval (at 0 35.56 270) (size 1.7 1.7) (drill 1) (layers "*.Cu" "*.Mask") (remove_unused_layers no) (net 12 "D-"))
  (pad "16" thru_hole oval (at 0 38.1 270) (size 1.7 1.7) (drill 1) (layers "*.Cu" "*.Mask") (remove_unused_layers no) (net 2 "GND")))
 (gr_arc (start 210 130) (mid 207.803301 135.303301) (end 202.5 137.5) (stroke (width 0.05) (type default)) (layer "Edge.Cuts"))
 (gr_arc (start 202.5 107.5) (mid 198.964466 106.035534) (end 197.5 102.5) (stroke (width 0.05) (type default)) (layer "Edge.Cuts"))
 (gr_line (start 197.5 97.5) (end 197.5 102.5) (stroke (width 0.05) (type default)) (layer "Edge.Cuts"))
 (gr_line (start 95 70) (end 95 87.5) (stroke (width 0.05) (type default)) (layer "Edge.Cuts"))
 (gr_line (start 202.5 62.5) (end 102.5 62.5) (stroke (width 0.05) (type default)) (layer "Edge.Cuts"))
 (gr_line (start 210 70) (end 210 87.5) (stroke (width 0.05) (type default)) (layer "Edge.Cuts"))
 (gr_line (start 107.5 97.5) (end 107.5 102.5) (stroke (width 0.05) (type default)) (layer "Edge.Cuts"))
 (gr_line (start 100 107.5) (end 102.5 107.5) (stroke (width 0.05) (type default)) (layer "Edge.Cuts"))
 (gr_circle (center 102.5 130) (end 104.1 130) (stroke (width 0.1) (type solid)) (fill no) (layer "Edge.Cuts"))
 (gr_arc (start 102.5 92.5) (mid 106.035534 93.964466) (end 107.5 97.5) (stroke (width 0.05) (type default)) (layer "Edge.Cuts"))
 (gr_circle (center 202.5 130) (end 204.1 130) (stroke (width 0.1) (type solid)) (fill no) (layer "Edge.Cuts"))
 (gr_arc (start 202.5 62.5) (mid 207.803301 64.696699) (end 210 70) (stroke (width 0.05) (type default)) (layer "Edge.Cuts"))
 (gr_arc (start 205 107.5) (mid 208.535534 108.964466) (end 210 112.5) (stroke (width 0.05) (type default)) (layer "Edge.Cuts"))
 (gr_line (start 210 112.5) (end 210 130) (stroke (width 0.05) (type default)) (layer "Edge.Cuts"))
 (gr_arc (start 197.5 97.5) (mid 198.964466 93.964466) (end 202.5 92.5) (stroke (width 0.05) (type default)) (layer "Edge.Cuts"))
 (gr_arc (start 107.5 102.5) (mid 106.035534 106.035534) (end 102.5 107.5) (stroke (width 0.05) (type default)) (layer "Edge.Cuts"))
 (gr_arc (start 95 112.5) (mid 96.464466 108.964466) (end 100 107.5) (stroke (width 0.05) (type default)) (layer "Edge.Cuts"))
 (gr_circle (center 102.5 70) (end 104.1 70) (stroke (width 0.1) (type solid)) (fill no) (layer "Edge.Cuts"))
 (gr_line (start 102.5 137.5) (end 202.5 137.5) (stroke (width 0.05) (type default)) (layer "Edge.Cuts"))
 (gr_line (start 205 92.5) (end 202.5 92.5) (stroke (width 0.05) (type default)) (layer "Edge.Cuts"))
 (gr_line (start 95 112.5) (end 95 130) (stroke (width 0.05) (type default)) (layer "Edge.Cuts"))
 (gr_arc (start 100 92.5) (mid 96.464466 91.035534) (end 95 87.5) (stroke (width 0.05) (type default)) (layer "Edge.Cuts"))
 (gr_arc (start 210 87.5) (mid 208.535534 91.035534) (end 205 92.5) (stroke (width 0.05) (type default)) (layer "Edge.Cuts"))
 (gr_line (start 100 92.5) (end 102.5 92.5) (stroke (width 0.05) (type default)) (layer "Edge.Cuts"))
 (gr_arc (start 95 70) (mid 97.196699 64.696699) (end 102.5 62.5) (stroke (width 0.05) (type default)) (layer "Edge.Cuts"))
 (gr_line (start 202.5 107.5) (end 205 107.5) (stroke (width 0.05) (type default)) (layer "Edge.Cuts"))
 (gr_circle (center 202.5 70) (end 204.1 70) (stroke (width 0.1) (type solid)) (fill no) (layer "Edge.Cuts"))
 (gr_arc (start 102.5 137.5) (mid 97.196699 135.303301) (end 95 130) (stroke (width 0.05) (type default)) (layer "Edge.Cuts"))
 (segment (start 187.543 66.7125) (end 194.5285 66.7125) (width 0.2) (layer "F.Cu") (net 2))
 (segment (start 186.367 67.8885) (end 187.543 66.7125) (width 0.2) (layer "F.Cu") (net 2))
 (segment (start 194.5285 66.7125) (end 196.262 68.446) (width 0.2) (layer "F.Cu") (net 2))
 (segment (start 194.7445 67.8885) (end 195.302 68.446) (width 0.2) (layer "F.Cu") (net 4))
 (segment (start 196.262 69.406) (end 195.302 68.446) (width 0.2) (layer "F.Cu") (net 4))
 (segment (start 196.262 72.256) (end 196.262 69.406) (width 0.2) (layer "F.Cu") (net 4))
 (segment (start 190.867 67.8885) (end 194.7445 67.8885) (width 0.2) (layer "F.Cu") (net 4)))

